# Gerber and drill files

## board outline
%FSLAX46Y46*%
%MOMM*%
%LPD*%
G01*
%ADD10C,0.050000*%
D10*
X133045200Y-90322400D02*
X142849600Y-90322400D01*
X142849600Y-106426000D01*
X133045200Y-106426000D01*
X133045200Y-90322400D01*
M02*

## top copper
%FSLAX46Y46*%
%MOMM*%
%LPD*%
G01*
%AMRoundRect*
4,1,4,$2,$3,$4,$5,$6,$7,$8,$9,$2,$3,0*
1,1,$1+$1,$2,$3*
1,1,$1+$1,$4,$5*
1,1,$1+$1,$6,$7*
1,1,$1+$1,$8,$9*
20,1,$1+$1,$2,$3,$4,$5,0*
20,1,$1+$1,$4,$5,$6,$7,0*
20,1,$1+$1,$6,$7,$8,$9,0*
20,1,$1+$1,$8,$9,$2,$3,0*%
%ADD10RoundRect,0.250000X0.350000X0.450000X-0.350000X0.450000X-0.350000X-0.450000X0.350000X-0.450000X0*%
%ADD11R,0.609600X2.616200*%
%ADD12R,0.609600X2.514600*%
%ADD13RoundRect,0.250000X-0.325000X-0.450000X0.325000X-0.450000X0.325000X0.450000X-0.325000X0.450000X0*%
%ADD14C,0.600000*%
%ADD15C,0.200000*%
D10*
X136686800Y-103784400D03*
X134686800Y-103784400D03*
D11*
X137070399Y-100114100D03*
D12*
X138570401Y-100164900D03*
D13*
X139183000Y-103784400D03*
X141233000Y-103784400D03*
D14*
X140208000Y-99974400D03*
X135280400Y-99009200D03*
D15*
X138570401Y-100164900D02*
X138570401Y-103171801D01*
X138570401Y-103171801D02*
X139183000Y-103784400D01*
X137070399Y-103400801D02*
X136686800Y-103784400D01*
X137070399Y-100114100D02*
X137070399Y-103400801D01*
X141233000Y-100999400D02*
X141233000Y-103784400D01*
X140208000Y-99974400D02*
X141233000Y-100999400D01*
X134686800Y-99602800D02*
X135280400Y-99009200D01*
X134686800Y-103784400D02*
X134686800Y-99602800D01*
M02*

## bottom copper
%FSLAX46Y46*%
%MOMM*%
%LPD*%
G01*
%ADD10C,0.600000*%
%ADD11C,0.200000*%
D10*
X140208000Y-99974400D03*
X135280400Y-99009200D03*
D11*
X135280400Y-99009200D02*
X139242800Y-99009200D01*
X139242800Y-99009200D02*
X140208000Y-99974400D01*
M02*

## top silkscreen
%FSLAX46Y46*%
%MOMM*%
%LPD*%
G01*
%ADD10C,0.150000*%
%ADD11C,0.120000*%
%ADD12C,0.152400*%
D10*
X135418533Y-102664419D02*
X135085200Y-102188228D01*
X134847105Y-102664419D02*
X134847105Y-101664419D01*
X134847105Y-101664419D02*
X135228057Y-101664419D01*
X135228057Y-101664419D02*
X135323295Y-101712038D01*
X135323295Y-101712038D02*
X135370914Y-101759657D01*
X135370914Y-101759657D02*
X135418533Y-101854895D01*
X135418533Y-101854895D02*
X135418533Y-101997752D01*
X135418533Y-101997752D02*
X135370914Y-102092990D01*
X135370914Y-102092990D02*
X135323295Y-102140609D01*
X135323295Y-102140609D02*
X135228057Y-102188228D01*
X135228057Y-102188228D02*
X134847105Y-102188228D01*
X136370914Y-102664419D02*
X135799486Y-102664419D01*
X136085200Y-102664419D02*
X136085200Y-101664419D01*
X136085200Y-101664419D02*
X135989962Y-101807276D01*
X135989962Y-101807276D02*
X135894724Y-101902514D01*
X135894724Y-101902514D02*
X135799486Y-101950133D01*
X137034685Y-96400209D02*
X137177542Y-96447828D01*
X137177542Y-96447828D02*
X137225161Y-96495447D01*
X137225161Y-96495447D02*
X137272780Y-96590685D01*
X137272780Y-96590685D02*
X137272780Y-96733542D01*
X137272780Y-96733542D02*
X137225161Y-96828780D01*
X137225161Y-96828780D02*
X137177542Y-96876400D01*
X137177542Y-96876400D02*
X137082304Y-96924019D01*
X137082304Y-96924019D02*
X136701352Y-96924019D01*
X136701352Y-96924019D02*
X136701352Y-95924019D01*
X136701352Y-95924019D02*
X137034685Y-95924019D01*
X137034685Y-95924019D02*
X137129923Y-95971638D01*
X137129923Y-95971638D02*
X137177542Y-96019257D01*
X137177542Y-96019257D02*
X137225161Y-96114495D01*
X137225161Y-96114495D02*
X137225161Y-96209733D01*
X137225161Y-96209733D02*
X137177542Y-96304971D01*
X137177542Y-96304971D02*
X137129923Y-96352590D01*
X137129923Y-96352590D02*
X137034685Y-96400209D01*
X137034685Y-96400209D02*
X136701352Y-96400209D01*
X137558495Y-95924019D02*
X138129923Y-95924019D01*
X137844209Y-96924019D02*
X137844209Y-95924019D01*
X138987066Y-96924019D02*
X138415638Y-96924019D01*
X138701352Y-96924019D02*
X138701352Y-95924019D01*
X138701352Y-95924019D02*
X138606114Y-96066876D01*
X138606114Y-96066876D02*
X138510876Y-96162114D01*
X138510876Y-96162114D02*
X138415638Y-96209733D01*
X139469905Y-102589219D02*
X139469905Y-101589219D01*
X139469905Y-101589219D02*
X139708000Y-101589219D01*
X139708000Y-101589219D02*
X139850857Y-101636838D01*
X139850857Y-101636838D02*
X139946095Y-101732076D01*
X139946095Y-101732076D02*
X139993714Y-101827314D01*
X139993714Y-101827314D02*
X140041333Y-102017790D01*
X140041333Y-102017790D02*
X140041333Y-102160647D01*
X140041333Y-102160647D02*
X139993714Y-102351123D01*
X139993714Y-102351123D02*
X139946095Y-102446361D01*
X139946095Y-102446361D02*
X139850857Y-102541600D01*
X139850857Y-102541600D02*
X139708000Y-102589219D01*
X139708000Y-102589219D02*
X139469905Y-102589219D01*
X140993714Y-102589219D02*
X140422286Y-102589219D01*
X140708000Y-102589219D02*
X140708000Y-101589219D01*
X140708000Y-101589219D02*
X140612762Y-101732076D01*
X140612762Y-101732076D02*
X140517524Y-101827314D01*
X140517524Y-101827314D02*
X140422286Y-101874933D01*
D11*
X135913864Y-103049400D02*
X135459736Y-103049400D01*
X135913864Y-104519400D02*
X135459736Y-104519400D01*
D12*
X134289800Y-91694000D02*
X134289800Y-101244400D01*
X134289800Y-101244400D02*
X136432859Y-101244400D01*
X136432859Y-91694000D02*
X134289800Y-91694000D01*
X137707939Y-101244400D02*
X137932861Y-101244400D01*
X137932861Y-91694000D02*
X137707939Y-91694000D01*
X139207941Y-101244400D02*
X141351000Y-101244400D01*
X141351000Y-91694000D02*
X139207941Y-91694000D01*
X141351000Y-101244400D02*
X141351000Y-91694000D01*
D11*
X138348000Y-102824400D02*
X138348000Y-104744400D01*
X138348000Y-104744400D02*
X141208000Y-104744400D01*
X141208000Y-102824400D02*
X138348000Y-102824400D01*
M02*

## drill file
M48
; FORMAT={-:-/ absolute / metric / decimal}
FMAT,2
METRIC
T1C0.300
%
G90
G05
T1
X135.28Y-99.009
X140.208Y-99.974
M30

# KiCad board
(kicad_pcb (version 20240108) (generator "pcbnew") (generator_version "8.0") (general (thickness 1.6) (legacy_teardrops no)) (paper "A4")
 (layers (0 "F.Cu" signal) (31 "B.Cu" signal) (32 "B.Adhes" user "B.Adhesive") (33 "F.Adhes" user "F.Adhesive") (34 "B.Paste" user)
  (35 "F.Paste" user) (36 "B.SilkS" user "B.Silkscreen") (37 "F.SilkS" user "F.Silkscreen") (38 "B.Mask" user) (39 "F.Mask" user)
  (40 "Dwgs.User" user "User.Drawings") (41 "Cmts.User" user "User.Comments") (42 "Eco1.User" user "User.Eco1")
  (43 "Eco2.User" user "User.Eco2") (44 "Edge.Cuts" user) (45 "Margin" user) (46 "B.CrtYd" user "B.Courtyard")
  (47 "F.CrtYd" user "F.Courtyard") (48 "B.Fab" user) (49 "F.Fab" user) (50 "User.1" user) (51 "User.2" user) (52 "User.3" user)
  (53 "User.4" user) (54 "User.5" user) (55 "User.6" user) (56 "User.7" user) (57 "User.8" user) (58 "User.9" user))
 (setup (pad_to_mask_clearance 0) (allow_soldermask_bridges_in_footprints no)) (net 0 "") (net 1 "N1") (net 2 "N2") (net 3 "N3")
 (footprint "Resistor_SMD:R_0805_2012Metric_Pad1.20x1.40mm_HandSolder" (layer "F.Cu") (at 135.6868 103.7844 180)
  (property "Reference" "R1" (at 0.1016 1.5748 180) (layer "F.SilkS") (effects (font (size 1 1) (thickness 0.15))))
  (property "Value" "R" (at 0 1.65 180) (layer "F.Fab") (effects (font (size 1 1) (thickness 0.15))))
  (fp_line (start -0.227064 0.735) (end 0.227064 0.735) (stroke (width 0.12) (type solid)) (layer "F.SilkS"))
  (fp_line (start -0.227064 -0.735) (end 0.227064 -0.735) (stroke (width 0.12) (type solid)) (layer "F.SilkS"))
  (pad "1" smd roundrect (at -1 0 180) (size 1.2 1.4) (layers "F.Cu" "F.Paste" "F.Mask") (roundrect_rratio 0.208333) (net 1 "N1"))
  (pad "2" smd roundrect (at 1 0 180) (size 1.2 1.4) (layers "F.Cu" "F.Paste" "F.Mask") (roundrect_rratio 0.208333) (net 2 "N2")))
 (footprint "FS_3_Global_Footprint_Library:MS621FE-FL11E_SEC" (layer "F.Cu") (at 137.8204 96.4692 90)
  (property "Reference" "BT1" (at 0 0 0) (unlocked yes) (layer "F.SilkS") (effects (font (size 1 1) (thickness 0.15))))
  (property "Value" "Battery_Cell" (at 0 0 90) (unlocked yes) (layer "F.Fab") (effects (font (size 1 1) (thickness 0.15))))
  (fp_line (start 4.7752 -3.5306) (end -4.7752 -3.5306) (stroke (width 0.1524) (type solid)) (layer "F.SilkS"))
  (fp_line (start -4.7752 -3.5306) (end -4.7752 -1.387541) (stroke (width 0.1524) (type solid)) (layer "F.SilkS"))
  (fp_line (start 4.7752 -1.387541) (end 4.7752 -3.5306) (stroke (width 0.1524) (type solid)) (layer "F.SilkS"))
  (fp_line (start -4.7752 -0.112461) (end -4.7752 0.112461) (stroke (width 0.1524) (type solid)) (layer "F.SilkS"))
  (fp_line (start 4.7752 0.112461) (end 4.7752 -0.112461) (stroke (width 0.1524) (type solid)) (layer "F.SilkS"))
  (fp_line (start -4.7752 1.387541) (end -4.7752 3.5306) (stroke (width 0.1524) (type solid)) (layer "F.SilkS"))
  (fp_line (start 4.7752 3.5306) (end 4.7752 1.387541) (stroke (width 0.1524) (type solid)) (layer "F.SilkS"))
  (fp_line (start -4.7752 3.5306) (end 4.7752 3.5306) (stroke (width 0.1524) (type solid)) (layer "F.SilkS"))
  (pad "1" smd rect (at -3.6449 -0.750001 90) (size 2.6162 0.6096) (layers "F.Cu" "F.Paste" "F.Mask") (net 1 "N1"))
  (pad "2" smd rect (at -3.6957 0.750001 90) (size 2.5146 0.6096) (layers "F.Cu" "F.Paste" "F.Mask") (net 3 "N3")))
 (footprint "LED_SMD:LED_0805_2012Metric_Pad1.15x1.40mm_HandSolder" (layer "F.Cu") (at 140.208 103.7844)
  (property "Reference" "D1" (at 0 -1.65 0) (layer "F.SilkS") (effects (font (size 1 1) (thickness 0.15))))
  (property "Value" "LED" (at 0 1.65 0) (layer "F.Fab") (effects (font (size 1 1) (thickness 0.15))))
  (fp_line (start -1.86 -0.96) (end -1.86 0.96) (stroke (width 0.12) (type solid)) (layer "F.SilkS"))
  (fp_line (start -1.86 0.96) (end 1 0.96) (stroke (width 0.12) (type solid)) (layer "F.SilkS"))
  (fp_line (start 1 -0.96) (end -1.86 -0.96) (stroke (width 0.12) (type solid)) (layer "F.SilkS"))
  (pad "1" smd roundrect (at -1.025 0) (size 1.15 1.4) (layers "F.Cu" "F.Paste" "F.Mask") (roundrect_rratio 0.217391) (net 3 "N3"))
  (pad "2" smd roundrect (at 1.025 0) (size 1.15 1.4) (layers "F.Cu" "F.Paste" "F.Mask") (roundrect_rratio 0.217391) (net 2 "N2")))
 (gr_rect (start 133.0452 90.3224) (end 142.8496 106.426) (stroke (width 0.05) (type default)) (fill none) (layer "Edge.Cuts"))
 (segment (start 138.570401 100.1649) (end 138.570401 103.171801) (width 0.2) (layer "F.Cu") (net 3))
 (segment (start 138.570401 103.171801) (end 139.183 103.7844) (width 0.2) (layer "F.Cu") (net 3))
 (segment (start 137.070399 103.400801) (end 136.6868 103.7844) (width 0.2) (layer "F.Cu") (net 1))
 (segment (start 137.070399 100.1141) (end 137.070399 103.400801) (width 0.2) (layer "F.Cu") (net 1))
 (segment (start 141.233 100.9994) (end 141.233 103.7844) (width 0.2) (layer "F.Cu") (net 2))
 (segment (start 140.208 99.9744) (end 141.233 100.9994) (width 0.2) (layer "F.Cu") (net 2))
 (segment (start 134.6868 99.6028) (end 135.2804 99.0092) (width 0.2) (layer "F.Cu") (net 2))
 (segment (start 134.6868 103.7844) (end 134.6868 99.6028) (width 0.2) (layer "F.Cu") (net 2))
 (via (at 140.208 99.9744) (size 0.6) (drill 0.3) (layers "F.Cu" "B.Cu") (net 2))
 (via (at 135.2804 99.0092) (size 0.6) (drill 0.3) (layers "F.Cu" "B.Cu") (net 2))
 (segment (start 135.2804 99.0092) (end 139.2428 99.0092) (width 0.2) (layer "B.Cu") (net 2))
 (segment (start 139.2428 99.0092) (end 140.208 99.9744) (width 0.2) (layer "B.Cu") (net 2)))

